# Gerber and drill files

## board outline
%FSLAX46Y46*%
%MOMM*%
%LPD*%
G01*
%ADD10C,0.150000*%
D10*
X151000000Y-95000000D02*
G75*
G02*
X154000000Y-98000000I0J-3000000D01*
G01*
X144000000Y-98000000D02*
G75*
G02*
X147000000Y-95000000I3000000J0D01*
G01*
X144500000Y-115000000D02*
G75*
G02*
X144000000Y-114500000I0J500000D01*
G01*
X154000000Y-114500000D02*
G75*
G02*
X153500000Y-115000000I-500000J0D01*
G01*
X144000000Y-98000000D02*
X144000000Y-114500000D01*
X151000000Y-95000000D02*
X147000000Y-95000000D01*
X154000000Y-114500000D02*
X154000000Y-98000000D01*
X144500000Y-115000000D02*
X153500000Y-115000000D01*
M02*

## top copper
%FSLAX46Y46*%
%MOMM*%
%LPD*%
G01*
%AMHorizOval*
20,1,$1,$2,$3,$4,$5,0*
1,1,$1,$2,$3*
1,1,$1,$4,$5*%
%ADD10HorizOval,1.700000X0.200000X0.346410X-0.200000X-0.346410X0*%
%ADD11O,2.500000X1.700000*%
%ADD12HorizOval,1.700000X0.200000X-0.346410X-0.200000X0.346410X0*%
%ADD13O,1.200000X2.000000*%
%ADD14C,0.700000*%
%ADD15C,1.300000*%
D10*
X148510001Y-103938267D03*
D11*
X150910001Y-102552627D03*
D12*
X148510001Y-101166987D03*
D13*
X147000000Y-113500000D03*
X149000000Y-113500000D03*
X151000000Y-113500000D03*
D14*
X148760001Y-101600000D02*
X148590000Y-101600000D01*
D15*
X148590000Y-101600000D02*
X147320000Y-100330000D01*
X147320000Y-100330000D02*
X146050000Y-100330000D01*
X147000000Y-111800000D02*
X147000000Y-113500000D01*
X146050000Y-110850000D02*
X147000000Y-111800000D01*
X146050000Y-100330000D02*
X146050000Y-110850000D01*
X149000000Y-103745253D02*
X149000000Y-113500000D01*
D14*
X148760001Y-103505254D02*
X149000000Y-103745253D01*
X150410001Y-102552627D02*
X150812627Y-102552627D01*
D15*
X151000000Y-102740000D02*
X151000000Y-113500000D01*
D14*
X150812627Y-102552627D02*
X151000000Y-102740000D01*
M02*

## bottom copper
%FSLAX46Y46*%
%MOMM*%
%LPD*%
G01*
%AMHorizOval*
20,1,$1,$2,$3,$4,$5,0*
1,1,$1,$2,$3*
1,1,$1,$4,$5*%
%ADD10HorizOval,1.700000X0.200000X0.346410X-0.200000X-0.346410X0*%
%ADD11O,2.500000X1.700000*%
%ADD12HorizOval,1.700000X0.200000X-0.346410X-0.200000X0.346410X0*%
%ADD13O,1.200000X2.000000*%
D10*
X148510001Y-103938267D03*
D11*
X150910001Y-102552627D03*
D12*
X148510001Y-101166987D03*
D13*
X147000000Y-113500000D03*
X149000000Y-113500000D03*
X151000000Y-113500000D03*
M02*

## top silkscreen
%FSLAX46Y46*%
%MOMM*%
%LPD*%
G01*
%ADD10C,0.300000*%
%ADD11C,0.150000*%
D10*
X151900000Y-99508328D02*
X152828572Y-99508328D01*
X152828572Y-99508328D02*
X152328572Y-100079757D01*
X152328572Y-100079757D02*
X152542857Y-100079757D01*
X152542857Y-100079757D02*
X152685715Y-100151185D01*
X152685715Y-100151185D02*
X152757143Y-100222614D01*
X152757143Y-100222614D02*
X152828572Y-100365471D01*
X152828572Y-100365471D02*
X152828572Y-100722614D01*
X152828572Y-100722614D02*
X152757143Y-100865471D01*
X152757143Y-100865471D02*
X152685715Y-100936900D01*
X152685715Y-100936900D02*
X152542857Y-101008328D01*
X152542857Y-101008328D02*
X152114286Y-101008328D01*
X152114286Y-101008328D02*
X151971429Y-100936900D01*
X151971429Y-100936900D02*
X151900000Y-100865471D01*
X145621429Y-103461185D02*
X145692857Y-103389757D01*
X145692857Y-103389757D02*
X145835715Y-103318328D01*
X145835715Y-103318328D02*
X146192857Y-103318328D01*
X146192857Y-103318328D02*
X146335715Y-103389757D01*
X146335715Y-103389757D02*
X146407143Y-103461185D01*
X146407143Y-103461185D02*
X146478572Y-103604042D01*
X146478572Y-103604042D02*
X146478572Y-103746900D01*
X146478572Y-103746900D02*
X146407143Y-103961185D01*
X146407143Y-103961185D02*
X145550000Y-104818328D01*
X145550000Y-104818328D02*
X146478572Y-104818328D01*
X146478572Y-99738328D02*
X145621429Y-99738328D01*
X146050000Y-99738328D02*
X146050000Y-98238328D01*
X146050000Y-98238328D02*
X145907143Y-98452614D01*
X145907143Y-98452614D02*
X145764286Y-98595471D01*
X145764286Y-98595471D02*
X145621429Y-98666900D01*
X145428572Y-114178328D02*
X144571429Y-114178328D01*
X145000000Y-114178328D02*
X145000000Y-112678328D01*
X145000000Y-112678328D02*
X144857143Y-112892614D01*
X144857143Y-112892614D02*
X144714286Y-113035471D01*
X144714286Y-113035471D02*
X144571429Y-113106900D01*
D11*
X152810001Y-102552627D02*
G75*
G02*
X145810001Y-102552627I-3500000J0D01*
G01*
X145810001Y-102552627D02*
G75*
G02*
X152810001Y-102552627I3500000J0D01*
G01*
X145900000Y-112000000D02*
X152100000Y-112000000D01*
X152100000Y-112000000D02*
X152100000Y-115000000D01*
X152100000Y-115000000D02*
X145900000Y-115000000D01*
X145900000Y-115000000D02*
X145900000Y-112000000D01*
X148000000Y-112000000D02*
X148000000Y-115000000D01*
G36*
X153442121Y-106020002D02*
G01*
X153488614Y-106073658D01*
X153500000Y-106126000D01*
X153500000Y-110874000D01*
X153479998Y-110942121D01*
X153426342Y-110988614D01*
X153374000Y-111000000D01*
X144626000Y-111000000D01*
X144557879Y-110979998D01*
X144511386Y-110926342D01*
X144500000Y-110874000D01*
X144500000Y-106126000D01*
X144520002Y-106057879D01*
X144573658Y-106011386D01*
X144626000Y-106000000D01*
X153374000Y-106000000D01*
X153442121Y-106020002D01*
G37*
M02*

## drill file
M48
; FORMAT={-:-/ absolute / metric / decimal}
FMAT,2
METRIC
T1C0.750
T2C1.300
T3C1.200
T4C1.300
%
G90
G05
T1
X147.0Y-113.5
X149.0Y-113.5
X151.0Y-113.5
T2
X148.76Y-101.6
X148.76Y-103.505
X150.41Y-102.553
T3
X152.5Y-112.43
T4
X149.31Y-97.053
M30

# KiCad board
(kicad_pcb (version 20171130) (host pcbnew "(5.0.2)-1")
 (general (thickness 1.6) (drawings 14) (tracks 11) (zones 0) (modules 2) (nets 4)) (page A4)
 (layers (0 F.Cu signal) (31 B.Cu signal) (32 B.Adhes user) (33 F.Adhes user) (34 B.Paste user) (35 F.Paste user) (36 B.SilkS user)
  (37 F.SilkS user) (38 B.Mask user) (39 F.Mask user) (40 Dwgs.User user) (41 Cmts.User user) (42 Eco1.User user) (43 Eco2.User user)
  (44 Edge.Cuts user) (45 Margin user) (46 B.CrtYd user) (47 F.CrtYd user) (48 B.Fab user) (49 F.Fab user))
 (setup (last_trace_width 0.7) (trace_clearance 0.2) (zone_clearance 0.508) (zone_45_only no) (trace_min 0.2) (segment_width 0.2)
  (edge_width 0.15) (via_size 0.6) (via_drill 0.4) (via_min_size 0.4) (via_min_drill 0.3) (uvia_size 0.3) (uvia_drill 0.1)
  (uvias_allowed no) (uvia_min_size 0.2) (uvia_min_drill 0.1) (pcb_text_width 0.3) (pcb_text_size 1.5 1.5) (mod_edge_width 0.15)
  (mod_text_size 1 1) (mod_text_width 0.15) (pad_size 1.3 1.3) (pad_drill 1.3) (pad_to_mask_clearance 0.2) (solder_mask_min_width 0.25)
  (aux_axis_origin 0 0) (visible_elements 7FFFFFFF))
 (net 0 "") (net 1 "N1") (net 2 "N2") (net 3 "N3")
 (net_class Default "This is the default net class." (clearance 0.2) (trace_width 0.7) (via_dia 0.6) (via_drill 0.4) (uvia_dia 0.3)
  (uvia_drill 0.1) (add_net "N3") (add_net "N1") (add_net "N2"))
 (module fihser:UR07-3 (layer F.Cu) (at 149.310001 102.552627)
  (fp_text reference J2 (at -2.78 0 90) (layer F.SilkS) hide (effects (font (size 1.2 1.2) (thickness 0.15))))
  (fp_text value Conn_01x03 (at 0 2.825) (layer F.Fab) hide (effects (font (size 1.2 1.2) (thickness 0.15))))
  (fp_circle (center 0 0) (end 0 3.5) (layer F.SilkS) (width 0.15))
  (pad "" np_thru_hole circle (at 0 -5.5 90) (size 1.3 1.3) (drill 1.3) (layers *.Cu *.Mask))
  (pad 2 thru_hole oval (at -0.55 0.952627 60) (size 2.5 1.7) (drill 1.3 (offset -0.5 0)) (layers *.Cu *.Mask) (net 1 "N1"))
  (pad 3 thru_hole oval (at 1.1 0) (size 2.5 1.7) (drill 1.3 (offset 0.5 0)) (layers *.Cu *.Mask) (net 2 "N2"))
  (pad 1 thru_hole oval (at -0.55 -0.952627 300) (size 2.5 1.7) (drill 1.3 (offset -0.5 0)) (layers *.Cu *.Mask) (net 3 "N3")))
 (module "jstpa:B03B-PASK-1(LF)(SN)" (layer F.Cu) (at 149 113.5)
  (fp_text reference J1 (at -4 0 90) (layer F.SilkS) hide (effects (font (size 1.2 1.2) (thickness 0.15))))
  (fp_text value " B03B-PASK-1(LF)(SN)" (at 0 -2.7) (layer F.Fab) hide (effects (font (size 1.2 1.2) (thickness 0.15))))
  (fp_line (start -3.1 -1.5) (end 3.1 -1.5) (layer F.SilkS) (width 0.15))
  (fp_line (start 3.1 -1.5) (end 3.1 1.5) (layer F.SilkS) (width 0.15))
  (fp_line (start 3.1 1.5) (end -3.1 1.5) (layer F.SilkS) (width 0.15))
  (fp_line (start -3.1 1.5) (end -3.1 -1.5) (layer F.SilkS) (width 0.15))
  (fp_line (start -1 -1.5) (end -1 1.5) (layer F.SilkS) (width 0.15))
  (pad 1 thru_hole oval (at -2 0) (size 1.2 2) (drill 0.75) (layers *.Cu *.Mask) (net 3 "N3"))
  (pad 2 thru_hole oval (at 0 0) (size 1.2 2) (drill 0.75) (layers *.Cu *.Mask) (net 1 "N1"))
  (pad 3 thru_hole oval (at 2 0) (size 1.2 2) (drill 0.75) (layers *.Cu *.Mask) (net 2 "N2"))
  (pad "" np_thru_hole circle (at 3.5 -1.07) (size 1.2 1.2) (drill 1.2) (layers *.Cu *.Mask)))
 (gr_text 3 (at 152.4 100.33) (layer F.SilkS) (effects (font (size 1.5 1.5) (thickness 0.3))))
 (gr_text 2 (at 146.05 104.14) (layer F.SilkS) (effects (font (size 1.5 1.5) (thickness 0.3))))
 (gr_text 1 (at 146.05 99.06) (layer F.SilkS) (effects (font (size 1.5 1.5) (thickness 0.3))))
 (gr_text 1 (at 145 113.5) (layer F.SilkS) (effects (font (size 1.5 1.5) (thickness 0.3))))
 (gr_arc (start 151 98) (end 151 95) (angle 90) (layer Edge.Cuts) (width 0.15))
 (gr_arc (start 147 98) (end 144 98) (angle 90) (layer Edge.Cuts) (width 0.15))
 (gr_arc (start 144.5 114.5) (end 144.5 115) (angle 90) (layer Edge.Cuts) (width 0.15))
 (gr_arc (start 153.5 114.5) (end 154 114.5) (angle 90) (layer Edge.Cuts) (width 0.15))
 (gr_line (start 144 98) (end 144 114.5) (layer Edge.Cuts) (width 0.15))
 (gr_line (start 151 95) (end 147 95) (layer Edge.Cuts) (width 0.15))
 (gr_line (start 154 114.5) (end 154 98) (layer Edge.Cuts) (width 0.15))
 (gr_line (start 144.5 115) (end 153.5 115) (layer Edge.Cuts) (width 0.15))
 (segment (start 148.760001 101.6) (end 148.59 101.6) (width 0.7) (layer F.Cu) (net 3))
 (segment (start 148.59 101.6) (end 147.32 100.33) (width 1.3) (layer F.Cu) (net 3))
 (segment (start 147.32 100.33) (end 146.05 100.33) (width 1.3) (layer F.Cu) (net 3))
 (segment (start 147 111.8) (end 147 113.5) (width 1.3) (layer F.Cu) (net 3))
 (segment (start 146.05 110.85) (end 147 111.8) (width 1.3) (layer F.Cu) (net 3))
 (segment (start 146.05 100.33) (end 146.05 110.85) (width 1.3) (layer F.Cu) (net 3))
 (segment (start 149 103.745253) (end 149 113.5) (width 1.3) (layer F.Cu) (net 1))
 (segment (start 148.760001 103.505254) (end 149 103.745253) (width 0.7) (layer F.Cu) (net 1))
 (segment (start 150.410001 102.552627) (end 150.812627 102.552627) (width 0.7) (layer F.Cu) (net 2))
 (segment (start 151 102.74) (end 151 113.5) (width 1.3) (layer F.Cu) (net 2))
 (segment (start 150.812627 102.552627) (end 151 102.74) (width 0.7) (layer F.Cu) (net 2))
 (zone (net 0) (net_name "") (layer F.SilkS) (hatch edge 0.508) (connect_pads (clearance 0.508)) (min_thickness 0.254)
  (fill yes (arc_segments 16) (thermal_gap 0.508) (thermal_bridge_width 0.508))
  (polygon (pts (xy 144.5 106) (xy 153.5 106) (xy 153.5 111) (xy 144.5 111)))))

